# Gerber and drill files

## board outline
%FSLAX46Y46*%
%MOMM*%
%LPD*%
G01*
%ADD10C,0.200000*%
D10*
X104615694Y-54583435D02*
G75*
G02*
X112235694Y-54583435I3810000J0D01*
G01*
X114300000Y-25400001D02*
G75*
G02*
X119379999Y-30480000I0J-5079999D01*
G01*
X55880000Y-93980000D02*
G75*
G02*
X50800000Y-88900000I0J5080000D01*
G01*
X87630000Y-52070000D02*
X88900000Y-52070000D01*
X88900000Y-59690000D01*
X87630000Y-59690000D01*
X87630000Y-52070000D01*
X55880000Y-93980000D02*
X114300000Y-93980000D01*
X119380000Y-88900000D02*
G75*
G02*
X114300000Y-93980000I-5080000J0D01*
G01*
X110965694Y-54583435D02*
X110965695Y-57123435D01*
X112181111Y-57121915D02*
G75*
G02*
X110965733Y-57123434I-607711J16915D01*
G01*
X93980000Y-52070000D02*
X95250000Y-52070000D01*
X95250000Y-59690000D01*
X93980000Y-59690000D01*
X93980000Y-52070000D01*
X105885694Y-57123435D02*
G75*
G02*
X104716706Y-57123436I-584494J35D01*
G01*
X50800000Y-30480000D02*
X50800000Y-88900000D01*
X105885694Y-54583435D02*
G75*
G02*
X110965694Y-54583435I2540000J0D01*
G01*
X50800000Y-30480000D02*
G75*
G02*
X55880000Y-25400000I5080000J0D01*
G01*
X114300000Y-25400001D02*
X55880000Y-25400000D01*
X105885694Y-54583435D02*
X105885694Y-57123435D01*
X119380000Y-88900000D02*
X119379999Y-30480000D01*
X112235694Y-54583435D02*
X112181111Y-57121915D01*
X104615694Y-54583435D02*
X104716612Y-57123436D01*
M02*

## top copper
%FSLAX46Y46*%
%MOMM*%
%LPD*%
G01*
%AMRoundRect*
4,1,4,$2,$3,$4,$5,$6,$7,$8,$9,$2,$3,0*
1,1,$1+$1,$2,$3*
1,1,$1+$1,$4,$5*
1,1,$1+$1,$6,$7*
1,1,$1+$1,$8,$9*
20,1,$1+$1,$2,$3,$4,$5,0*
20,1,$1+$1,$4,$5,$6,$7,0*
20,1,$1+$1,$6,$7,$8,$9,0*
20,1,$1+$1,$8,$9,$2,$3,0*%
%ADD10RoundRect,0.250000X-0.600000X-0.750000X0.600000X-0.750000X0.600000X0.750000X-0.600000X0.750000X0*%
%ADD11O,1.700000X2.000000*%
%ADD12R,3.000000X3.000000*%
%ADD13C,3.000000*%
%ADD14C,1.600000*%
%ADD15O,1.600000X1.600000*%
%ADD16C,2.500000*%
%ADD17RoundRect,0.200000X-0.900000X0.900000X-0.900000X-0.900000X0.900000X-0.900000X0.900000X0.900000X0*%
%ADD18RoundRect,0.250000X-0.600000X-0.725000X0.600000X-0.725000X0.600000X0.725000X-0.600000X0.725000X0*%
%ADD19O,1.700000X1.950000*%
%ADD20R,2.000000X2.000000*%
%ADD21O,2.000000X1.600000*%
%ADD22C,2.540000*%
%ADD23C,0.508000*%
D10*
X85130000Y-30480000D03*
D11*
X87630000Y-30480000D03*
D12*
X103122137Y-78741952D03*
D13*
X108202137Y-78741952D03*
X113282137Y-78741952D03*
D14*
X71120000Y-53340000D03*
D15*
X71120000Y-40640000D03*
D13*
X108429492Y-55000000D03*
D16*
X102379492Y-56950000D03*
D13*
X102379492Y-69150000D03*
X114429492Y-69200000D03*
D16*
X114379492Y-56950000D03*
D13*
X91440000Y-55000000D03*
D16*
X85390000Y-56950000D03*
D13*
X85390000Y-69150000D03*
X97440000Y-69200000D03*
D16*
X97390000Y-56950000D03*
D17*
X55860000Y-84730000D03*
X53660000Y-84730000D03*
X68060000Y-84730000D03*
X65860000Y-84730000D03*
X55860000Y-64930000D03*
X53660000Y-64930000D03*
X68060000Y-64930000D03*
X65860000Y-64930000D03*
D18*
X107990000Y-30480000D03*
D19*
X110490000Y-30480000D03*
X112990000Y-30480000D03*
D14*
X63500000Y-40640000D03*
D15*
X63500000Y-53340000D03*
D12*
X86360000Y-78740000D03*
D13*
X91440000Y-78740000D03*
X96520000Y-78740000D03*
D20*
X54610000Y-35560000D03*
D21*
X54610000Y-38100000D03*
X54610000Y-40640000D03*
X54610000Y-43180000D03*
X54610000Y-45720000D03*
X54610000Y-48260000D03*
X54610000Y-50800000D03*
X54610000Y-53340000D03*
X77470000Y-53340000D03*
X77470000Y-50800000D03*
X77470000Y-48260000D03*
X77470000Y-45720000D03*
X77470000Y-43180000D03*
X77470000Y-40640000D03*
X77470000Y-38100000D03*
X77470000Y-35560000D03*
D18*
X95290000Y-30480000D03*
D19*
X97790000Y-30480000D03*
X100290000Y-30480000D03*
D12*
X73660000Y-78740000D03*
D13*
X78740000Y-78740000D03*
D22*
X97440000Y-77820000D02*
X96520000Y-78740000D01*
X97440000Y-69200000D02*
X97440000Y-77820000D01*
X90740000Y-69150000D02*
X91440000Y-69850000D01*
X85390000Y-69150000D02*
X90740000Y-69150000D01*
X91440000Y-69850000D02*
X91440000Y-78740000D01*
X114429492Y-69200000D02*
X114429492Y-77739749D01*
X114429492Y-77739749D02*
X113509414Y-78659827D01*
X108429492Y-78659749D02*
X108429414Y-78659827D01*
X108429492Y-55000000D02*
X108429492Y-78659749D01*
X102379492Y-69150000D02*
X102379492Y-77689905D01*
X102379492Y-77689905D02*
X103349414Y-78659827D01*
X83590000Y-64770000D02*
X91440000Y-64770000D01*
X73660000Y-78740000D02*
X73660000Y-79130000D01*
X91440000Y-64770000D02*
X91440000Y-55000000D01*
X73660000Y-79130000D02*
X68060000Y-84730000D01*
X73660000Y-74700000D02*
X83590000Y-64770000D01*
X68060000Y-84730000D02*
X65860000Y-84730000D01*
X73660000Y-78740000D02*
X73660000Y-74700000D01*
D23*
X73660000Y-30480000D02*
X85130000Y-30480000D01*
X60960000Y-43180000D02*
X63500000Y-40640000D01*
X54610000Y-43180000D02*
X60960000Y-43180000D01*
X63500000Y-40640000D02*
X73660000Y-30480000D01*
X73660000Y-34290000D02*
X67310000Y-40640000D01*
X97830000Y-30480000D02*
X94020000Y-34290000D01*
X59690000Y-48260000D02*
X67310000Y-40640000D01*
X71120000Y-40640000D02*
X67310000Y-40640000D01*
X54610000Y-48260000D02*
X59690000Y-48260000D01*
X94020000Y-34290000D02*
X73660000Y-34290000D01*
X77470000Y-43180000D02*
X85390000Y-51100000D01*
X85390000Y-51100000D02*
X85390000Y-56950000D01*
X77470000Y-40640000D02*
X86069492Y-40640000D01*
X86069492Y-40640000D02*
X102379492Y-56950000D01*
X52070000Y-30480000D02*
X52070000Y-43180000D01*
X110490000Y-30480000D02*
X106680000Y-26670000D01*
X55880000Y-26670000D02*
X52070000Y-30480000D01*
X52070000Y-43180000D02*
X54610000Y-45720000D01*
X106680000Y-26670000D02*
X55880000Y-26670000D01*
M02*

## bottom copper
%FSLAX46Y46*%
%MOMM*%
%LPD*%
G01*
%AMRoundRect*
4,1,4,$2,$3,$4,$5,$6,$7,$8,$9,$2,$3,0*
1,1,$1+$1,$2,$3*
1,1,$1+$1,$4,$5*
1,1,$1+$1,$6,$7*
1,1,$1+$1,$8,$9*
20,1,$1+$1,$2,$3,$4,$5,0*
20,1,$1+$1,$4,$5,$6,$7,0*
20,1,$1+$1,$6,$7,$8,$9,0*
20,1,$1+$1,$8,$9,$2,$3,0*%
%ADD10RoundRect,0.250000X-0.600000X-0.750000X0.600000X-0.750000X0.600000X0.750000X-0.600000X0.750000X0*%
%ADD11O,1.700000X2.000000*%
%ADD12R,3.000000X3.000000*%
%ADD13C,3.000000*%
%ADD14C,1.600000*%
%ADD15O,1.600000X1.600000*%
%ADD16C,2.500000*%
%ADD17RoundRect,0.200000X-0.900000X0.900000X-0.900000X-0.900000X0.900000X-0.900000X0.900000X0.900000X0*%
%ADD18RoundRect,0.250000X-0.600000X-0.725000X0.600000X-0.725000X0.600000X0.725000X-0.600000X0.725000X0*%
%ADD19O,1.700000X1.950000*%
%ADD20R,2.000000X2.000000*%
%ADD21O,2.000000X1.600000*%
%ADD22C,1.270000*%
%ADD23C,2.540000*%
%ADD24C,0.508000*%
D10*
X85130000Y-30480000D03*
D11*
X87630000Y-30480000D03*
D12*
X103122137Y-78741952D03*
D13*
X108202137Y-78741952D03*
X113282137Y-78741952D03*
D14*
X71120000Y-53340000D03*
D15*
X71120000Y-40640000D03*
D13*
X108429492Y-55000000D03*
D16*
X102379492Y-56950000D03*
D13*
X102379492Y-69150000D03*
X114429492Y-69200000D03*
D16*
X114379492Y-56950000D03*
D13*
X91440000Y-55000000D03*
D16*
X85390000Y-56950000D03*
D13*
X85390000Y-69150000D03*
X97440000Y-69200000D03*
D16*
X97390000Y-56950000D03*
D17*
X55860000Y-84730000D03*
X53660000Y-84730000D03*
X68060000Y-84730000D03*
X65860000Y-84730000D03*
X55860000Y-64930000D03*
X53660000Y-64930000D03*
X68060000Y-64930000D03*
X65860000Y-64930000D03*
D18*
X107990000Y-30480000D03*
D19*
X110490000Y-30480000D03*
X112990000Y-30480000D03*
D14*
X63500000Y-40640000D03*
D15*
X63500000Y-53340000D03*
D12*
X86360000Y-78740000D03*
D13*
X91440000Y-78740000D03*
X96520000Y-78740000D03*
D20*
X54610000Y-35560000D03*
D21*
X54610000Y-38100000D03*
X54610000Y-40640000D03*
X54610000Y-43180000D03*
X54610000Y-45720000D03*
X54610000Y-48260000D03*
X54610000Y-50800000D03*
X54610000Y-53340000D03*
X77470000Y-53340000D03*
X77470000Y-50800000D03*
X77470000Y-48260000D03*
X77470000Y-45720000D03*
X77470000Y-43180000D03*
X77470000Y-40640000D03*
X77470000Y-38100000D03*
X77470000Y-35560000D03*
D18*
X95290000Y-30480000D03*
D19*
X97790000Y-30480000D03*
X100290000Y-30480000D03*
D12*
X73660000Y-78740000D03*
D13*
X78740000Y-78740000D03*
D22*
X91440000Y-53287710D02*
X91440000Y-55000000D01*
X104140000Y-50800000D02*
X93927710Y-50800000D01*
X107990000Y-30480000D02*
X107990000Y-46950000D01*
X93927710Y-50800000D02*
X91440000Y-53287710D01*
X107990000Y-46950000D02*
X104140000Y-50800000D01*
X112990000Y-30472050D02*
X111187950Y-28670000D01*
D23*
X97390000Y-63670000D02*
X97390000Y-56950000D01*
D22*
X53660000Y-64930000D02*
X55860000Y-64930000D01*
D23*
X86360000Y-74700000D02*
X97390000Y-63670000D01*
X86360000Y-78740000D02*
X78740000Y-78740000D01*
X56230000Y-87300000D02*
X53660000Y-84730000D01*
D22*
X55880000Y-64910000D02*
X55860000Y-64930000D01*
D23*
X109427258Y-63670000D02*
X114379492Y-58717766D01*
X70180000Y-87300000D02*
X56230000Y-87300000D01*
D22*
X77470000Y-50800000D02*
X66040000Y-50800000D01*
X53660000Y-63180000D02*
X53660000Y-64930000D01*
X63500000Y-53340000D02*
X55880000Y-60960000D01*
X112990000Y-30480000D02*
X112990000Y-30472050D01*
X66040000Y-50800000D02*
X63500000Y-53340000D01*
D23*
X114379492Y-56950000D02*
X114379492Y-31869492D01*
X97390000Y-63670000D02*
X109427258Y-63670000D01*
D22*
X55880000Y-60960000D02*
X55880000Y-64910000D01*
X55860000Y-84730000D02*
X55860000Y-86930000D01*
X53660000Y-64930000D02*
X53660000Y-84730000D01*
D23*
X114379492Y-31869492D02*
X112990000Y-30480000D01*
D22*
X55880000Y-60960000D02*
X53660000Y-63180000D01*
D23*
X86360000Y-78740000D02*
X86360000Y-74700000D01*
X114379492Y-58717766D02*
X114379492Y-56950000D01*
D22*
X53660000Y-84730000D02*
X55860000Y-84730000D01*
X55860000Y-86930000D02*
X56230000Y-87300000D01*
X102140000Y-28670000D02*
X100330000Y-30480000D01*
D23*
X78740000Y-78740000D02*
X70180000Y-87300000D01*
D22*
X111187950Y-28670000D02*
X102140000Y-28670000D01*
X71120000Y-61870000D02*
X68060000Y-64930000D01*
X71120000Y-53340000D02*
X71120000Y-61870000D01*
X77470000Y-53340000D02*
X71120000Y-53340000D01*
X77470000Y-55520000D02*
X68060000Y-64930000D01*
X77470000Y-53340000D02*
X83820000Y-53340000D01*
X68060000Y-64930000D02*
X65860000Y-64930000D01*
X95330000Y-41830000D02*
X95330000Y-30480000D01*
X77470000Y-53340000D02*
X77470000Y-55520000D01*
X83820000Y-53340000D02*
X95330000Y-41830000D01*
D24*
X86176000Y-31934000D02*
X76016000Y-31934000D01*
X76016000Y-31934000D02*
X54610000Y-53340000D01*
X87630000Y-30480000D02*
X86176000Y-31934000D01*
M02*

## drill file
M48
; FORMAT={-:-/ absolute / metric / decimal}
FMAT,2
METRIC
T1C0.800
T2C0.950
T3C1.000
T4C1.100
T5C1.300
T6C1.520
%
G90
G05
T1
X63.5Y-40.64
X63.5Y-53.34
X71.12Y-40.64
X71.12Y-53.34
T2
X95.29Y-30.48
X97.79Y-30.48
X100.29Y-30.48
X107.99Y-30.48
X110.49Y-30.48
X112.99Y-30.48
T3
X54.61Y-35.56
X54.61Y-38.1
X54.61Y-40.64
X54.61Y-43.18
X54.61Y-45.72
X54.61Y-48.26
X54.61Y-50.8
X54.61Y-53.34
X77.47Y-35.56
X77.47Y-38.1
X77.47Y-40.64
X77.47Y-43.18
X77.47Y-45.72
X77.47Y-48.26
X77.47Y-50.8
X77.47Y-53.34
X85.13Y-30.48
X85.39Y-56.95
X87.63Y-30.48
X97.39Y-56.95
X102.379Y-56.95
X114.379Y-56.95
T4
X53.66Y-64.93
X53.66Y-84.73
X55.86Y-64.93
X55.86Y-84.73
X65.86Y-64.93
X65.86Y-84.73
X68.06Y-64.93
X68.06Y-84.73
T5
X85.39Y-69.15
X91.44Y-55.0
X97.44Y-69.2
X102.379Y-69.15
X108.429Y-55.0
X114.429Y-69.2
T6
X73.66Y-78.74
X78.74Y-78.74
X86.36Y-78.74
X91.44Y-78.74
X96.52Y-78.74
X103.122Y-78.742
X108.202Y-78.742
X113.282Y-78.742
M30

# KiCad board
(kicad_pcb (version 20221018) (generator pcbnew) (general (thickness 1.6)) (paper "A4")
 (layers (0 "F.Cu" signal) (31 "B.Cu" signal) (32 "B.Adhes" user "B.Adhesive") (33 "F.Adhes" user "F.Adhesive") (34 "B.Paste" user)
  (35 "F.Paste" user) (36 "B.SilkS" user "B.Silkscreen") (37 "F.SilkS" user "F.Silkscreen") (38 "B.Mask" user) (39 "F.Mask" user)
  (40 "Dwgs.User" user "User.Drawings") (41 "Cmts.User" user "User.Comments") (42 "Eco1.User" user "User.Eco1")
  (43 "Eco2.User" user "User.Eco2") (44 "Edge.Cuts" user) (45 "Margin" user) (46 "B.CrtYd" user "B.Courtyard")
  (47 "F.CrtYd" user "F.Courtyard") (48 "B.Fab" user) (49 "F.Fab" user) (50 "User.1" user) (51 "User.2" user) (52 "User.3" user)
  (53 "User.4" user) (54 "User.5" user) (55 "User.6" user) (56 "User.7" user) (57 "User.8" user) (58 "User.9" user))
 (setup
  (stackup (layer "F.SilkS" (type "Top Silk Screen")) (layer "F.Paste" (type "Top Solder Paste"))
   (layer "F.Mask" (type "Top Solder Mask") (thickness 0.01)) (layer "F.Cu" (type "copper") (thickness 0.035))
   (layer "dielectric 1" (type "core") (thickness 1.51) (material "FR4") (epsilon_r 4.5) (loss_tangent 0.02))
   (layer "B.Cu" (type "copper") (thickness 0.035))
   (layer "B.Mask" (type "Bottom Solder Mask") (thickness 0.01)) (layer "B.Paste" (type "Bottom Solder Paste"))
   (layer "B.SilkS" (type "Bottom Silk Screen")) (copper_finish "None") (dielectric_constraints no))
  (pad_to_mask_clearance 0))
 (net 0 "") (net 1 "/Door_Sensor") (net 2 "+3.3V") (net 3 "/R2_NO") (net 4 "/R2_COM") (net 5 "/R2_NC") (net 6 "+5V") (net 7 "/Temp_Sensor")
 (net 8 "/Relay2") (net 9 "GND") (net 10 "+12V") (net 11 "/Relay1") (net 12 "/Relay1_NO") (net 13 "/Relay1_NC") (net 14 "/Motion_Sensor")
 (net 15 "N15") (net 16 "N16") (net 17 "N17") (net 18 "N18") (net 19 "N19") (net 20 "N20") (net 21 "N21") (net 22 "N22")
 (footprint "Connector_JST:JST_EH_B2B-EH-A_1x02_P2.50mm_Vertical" (layer "F.Cu") (at 85.13 30.48)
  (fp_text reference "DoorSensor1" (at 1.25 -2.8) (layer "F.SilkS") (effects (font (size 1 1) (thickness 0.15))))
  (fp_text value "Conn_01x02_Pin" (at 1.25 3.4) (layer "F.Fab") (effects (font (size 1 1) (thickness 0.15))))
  (pad "1" thru_hole roundrect (at 0 0) (size 1.7 2) (drill 1) (layers "*.Cu" "*.Mask") (roundrect_rratio 0.1470588235)
   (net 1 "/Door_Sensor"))
  (pad "2" thru_hole oval (at 2.5 0) (size 1.7 2) (drill 1) (layers "*.Cu" "*.Mask") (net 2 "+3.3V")))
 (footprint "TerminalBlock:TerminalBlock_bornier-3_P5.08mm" (layer "F.Cu") (at 103.122137 78.741952)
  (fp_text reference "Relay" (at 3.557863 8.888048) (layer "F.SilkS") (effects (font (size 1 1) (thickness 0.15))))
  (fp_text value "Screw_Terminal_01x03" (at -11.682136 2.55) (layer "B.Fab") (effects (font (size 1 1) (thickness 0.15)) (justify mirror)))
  (pad "1" thru_hole rect (at 0 0) (size 3 3) (drill 1.52) (layers "*.Cu" "*.Mask") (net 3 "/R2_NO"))
  (pad "2" thru_hole circle (at 5.08 0) (size 3 3) (drill 1.52) (layers "*.Cu" "*.Mask") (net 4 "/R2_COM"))
  (pad "3" thru_hole circle (at 10.16 0) (size 3 3) (drill 1.52) (layers "*.Cu" "*.Mask") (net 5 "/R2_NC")))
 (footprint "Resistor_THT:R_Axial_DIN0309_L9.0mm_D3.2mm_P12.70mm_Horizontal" (layer "F.Cu") (at 71.12 53.34 90)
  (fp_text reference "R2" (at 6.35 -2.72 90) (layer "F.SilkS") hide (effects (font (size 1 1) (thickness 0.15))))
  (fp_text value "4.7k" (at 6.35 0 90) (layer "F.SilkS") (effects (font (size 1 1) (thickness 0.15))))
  (pad "1" thru_hole circle (at 0 0 90) (size 1.6 1.6) (drill 0.8) (layers "*.Cu" "*.Mask") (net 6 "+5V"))
  (pad "2" thru_hole oval (at 12.7 0 90) (size 1.6 1.6) (drill 0.8) (layers "*.Cu" "*.Mask") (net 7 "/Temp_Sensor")))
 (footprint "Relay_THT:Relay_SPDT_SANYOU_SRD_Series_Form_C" (layer "F.Cu") (at 108.429492 55 -90)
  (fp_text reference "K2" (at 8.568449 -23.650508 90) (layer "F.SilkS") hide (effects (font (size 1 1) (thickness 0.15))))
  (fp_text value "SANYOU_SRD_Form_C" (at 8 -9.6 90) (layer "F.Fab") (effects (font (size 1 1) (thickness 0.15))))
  (pad "1" thru_hole circle (at 0 0) (size 3 3) (drill 1.3) (layers "*.Cu" "*.Mask") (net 4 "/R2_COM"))
  (pad "2" thru_hole circle (at 1.95 6.05) (size 2.5 2.5) (drill 1) (layers "*.Cu" "*.Mask") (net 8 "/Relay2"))
  (pad "3" thru_hole circle (at 14.15 6.05) (size 3 3) (drill 1.3) (layers "*.Cu" "*.Mask") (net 3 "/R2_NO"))
  (pad "4" thru_hole circle (at 14.2 -6) (size 3 3) (drill 1.3) (layers "*.Cu" "*.Mask") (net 5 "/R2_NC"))
  (pad "5" thru_hole circle (at 1.95 -5.95) (size 2.5 2.5) (drill 1) (layers "*.Cu" "*.Mask") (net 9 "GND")))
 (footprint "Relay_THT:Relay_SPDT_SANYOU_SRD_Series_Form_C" (layer "F.Cu") (at 91.44 55 -90)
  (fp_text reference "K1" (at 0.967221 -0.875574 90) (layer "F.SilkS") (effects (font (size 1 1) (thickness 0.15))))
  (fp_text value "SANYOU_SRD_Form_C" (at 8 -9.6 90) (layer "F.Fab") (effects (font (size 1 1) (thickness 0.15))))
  (pad "1" thru_hole circle (at 0 0) (size 3 3) (drill 1.3) (layers "*.Cu" "*.Mask") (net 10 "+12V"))
  (pad "2" thru_hole circle (at 1.95 6.05) (size 2.5 2.5) (drill 1) (layers "*.Cu" "*.Mask") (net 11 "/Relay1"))
  (pad "3" thru_hole circle (at 14.15 6.05) (size 3 3) (drill 1.3) (layers "*.Cu" "*.Mask") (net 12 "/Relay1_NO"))
  (pad "4" thru_hole circle (at 14.2 -6) (size 3 3) (drill 1.3) (layers "*.Cu" "*.Mask") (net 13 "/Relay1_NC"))
  (pad "5" thru_hole circle (at 1.95 -5.95) (size 2.5 2.5) (drill 1) (layers "*.Cu" "*.Mask") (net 9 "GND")))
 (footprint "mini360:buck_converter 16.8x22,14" (layer "F.Cu") (at 60.96 74.93 -90)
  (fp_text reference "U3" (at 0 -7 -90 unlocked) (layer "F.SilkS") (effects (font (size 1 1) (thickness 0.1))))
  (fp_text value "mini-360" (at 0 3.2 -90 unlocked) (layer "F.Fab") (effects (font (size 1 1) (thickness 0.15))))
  (pad "1" thru_hole roundrect (at 9.8 5.1 270) (size 2.2 2.2) (drill 1.1) (layers "*.Cu" "*.Mask") (roundrect_rratio 0.09090909091)
   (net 9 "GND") (thermal_bridge_angle 45))
  (pad "1" thru_hole roundrect (at 9.8 7.3 270) (size 2.2 2.2) (drill 1.1) (layers "*.Cu" "*.Mask") (roundrect_rratio 0.09090909091)
   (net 9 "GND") (thermal_bridge_angle 45))
  (pad "2" thru_hole roundrect (at 9.8 -7.1 270) (size 2.2 2.2) (drill 1.1) (layers "*.Cu" "*.Mask") (roundrect_rratio 0.09090909091)
   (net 10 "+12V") (thermal_bridge_angle 45))
  (pad "2" thru_hole roundrect (at 9.8 -4.9 270) (size 2.2 2.2) (drill 1.1) (layers "*.Cu" "*.Mask") (roundrect_rratio 0.09090909091)
   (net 10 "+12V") (thermal_bridge_angle 45))
  (pad "3" thru_hole roundrect (at -10 5.1 270) (size 2.2 2.2) (drill 1.1) (layers "*.Cu" "*.Mask") (roundrect_rratio 0.09090909091)
   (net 9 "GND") (thermal_bridge_angle 45))
  (pad "3" thru_hole roundrect (at -10 7.3 270) (size 2.2 2.2) (drill 1.1) (layers "*.Cu" "*.Mask") (roundrect_rratio 0.09090909091)
   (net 9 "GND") (thermal_bridge_angle 45))
  (pad "4" thru_hole roundrect (at -10 -7.1 270) (size 2.2 2.2) (drill 1.1) (layers "*.Cu" "*.Mask") (roundrect_rratio 0.09090909091)
   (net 6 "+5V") (thermal_bridge_angle 45))
  (pad "4" thru_hole roundrect (at -10 -4.9 270) (size 2.2 2.2) (drill 1.1) (layers "*.Cu" "*.Mask") (roundrect_rratio 0.09090909091)
   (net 6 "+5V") (thermal_bridge_angle 45)))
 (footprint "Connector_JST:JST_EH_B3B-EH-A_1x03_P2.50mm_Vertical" (layer "F.Cu") (at 107.99 30.48)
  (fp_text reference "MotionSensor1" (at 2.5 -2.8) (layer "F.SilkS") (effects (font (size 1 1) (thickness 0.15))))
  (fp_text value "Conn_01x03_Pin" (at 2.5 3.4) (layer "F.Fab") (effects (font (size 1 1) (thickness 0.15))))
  (pad "1" thru_hole roundrect (at 0 0) (size 1.7 1.95) (drill 0.95) (layers "*.Cu" "*.Mask") (roundrect_rratio 0.1470588235)
   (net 10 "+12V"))
  (pad "2" thru_hole oval (at 2.5 0) (size 1.7 1.95) (drill 0.95) (layers "*.Cu" "*.Mask") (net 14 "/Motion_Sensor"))
  (pad "3" thru_hole oval (at 5 0) (size 1.7 1.95) (drill 0.95) (layers "*.Cu" "*.Mask") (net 9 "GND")))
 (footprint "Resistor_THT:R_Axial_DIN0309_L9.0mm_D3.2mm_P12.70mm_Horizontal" (layer "F.Cu") (at 63.5 40.64 -90)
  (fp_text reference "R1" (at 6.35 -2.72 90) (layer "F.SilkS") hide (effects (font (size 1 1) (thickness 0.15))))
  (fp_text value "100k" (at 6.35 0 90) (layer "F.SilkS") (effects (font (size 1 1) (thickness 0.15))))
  (pad "1" thru_hole circle (at 0 0 270) (size 1.6 1.6) (drill 0.8) (layers "*.Cu" "*.Mask") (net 1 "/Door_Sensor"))
  (pad "2" thru_hole oval (at 12.7 0 270) (size 1.6 1.6) (drill 0.8) (layers "*.Cu" "*.Mask") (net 9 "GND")))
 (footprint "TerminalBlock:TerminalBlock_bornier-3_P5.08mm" (layer "F.Cu") (at 86.36 78.74)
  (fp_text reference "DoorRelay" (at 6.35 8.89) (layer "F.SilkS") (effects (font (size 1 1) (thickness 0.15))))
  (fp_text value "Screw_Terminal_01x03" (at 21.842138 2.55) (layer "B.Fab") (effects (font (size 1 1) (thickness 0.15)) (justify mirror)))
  (pad "1" thru_hole rect (at 0 0) (size 3 3) (drill 1.52) (layers "*.Cu" "*.Mask") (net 9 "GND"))
  (pad "2" thru_hole circle (at 5.08 0) (size 3 3) (drill 1.52) (layers "*.Cu" "*.Mask") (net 12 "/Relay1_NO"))
  (pad "3" thru_hole circle (at 10.16 0) (size 3 3) (drill 1.52) (layers "*.Cu" "*.Mask") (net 13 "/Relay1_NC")))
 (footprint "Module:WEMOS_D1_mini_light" (layer "F.Cu") (at 54.61 35.56)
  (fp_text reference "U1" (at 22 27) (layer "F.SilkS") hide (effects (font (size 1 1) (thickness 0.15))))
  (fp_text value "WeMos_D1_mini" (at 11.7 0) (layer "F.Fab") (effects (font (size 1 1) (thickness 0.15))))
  (pad "1" thru_hole rect (at 0 0) (size 2 2) (drill 1) (layers "*.Cu" "*.Mask") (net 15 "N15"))
  (pad "2" thru_hole oval (at 0 2.54) (size 2 1.6) (drill 1) (layers "*.Cu" "*.Mask") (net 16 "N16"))
  (pad "3" thru_hole oval (at 0 5.08) (size 2 1.6) (drill 1) (layers "*.Cu" "*.Mask") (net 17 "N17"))
  (pad "4" thru_hole oval (at 0 7.62) (size 2 1.6) (drill 1) (layers "*.Cu" "*.Mask") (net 1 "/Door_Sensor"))
  (pad "5" thru_hole oval (at 0 10.16) (size 2 1.6) (drill 1) (layers "*.Cu" "*.Mask") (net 14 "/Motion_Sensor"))
  (pad "6" thru_hole oval (at 0 12.7) (size 2 1.6) (drill 1) (layers "*.Cu" "*.Mask") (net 7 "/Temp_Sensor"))
  (pad "7" thru_hole oval (at 0 15.24) (size 2 1.6) (drill 1) (layers "*.Cu" "*.Mask") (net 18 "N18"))
  (pad "8" thru_hole oval (at 0 17.78) (size 2 1.6) (drill 1) (layers "*.Cu" "*.Mask") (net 2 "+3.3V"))
  (pad "9" thru_hole oval (at 22.86 17.78) (size 2 1.6) (drill 1) (layers "*.Cu" "*.Mask") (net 6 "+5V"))
  (pad "10" thru_hole oval (at 22.86 15.24) (size 2 1.6) (drill 1) (layers "*.Cu" "*.Mask") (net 9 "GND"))
  (pad "11" thru_hole oval (at 22.86 12.7) (size 2 1.6) (drill 1) (layers "*.Cu" "*.Mask") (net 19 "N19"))
  (pad "12" thru_hole oval (at 22.86 10.16) (size 2 1.6) (drill 1) (layers "*.Cu" "*.Mask") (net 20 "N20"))
  (pad "13" thru_hole oval (at 22.86 7.62) (size 2 1.6) (drill 1) (layers "*.Cu" "*.Mask") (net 11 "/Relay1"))
  (pad "14" thru_hole oval (at 22.86 5.08) (size 2 1.6) (drill 1) (layers "*.Cu" "*.Mask") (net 8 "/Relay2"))
  (pad "15" thru_hole oval (at 22.86 2.54) (size 2 1.6) (drill 1) (layers "*.Cu" "*.Mask") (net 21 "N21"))
  (pad "16" thru_hole oval (at 22.86 0) (size 2 1.6) (drill 1) (layers "*.Cu" "*.Mask") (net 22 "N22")))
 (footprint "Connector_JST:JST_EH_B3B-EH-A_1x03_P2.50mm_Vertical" (layer "F.Cu") (at 95.29 30.48)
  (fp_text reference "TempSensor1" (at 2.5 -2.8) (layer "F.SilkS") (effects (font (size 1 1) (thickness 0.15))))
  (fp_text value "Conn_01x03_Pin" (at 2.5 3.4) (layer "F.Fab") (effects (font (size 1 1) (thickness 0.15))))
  (pad "1" thru_hole roundrect (at 0 0) (size 1.7 1.95) (drill 0.95) (layers "*.Cu" "*.Mask") (roundrect_rratio 0.1470588235) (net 6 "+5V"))
  (pad "2" thru_hole oval (at 2.5 0) (size 1.7 1.95) (drill 0.95) (layers "*.Cu" "*.Mask") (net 7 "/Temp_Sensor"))
  (pad "3" thru_hole oval (at 5 0) (size 1.7 1.95) (drill 0.95) (layers "*.Cu" "*.Mask") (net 9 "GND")))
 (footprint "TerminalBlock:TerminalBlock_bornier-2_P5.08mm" (layer "F.Cu") (at 73.66 78.74)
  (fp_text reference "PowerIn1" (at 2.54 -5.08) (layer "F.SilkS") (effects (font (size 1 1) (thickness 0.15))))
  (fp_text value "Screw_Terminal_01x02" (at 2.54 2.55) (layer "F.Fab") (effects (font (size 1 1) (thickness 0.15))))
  (pad "1" thru_hole rect (at 0 0) (size 3 3) (drill 1.52) (layers "*.Cu" "*.Mask") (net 10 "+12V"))
  (pad "2" thru_hole circle (at 5.08 0) (size 3 3) (drill 1.52) (layers "*.Cu" "*.Mask") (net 9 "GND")))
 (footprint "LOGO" (layer "B.Cu") (at 67.31 59.69 180)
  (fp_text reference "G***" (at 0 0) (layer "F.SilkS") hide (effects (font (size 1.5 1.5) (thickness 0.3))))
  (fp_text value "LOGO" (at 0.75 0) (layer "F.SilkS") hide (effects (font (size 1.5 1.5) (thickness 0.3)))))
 (gr_arc (start 104.615694 54.583435) (mid 108.425694 50.773435) (end 112.235694 54.583435) (stroke (width 0.2) (type default))
  (layer "Edge.Cuts"))
 (gr_arc (start 114.3 25.400001) (mid 117.892102 26.887898) (end 119.379999 30.48) (stroke (width 0.2) (type default)) (layer "Edge.Cuts"))
 (gr_arc (start 55.88 93.98) (mid 52.287898 92.492102) (end 50.8 88.9) (stroke (width 0.2) (type default)) (layer "Edge.Cuts"))
 (gr_rect (start 87.63 52.07) (end 88.9 59.69) (stroke (width 0.2) (type default)) (fill none) (layer "Edge.Cuts"))
 (gr_line (start 55.88 93.98) (end 114.3 93.98) (stroke (width 0.2) (type default)) (layer "Edge.Cuts"))
 (gr_arc (start 119.38 88.9) (mid 117.892102 92.492102) (end 114.3 93.98) (stroke (width 0.2) (type default)) (layer "Edge.Cuts"))
 (gr_line (start 110.965694 54.583435) (end 110.965695 57.123435) (stroke (width 0.2) (type default)) (layer "Edge.Cuts"))
 (gr_arc (start 112.181111 57.121915) (mid 111.574141 57.712966) (end 110.965695 57.123435) (stroke (width 0.2) (type default))
  (layer "Edge.Cuts"))
 (gr_rect (start 93.98 52.07) (end 95.25 59.69) (stroke (width 0.2) (type default)) (fill none) (layer "Edge.Cuts"))
 (gr_arc (start 105.885694 57.123435) (mid 105.301153 57.707941) (end 104.716612 57.123436) (stroke (width 0.2) (type default))
  (layer "Edge.Cuts"))
 (gr_line (start 50.8 30.48) (end 50.8 88.9) (stroke (width 0.2) (type default)) (layer "Edge.Cuts"))
 (gr_arc (start 105.885694 54.583435) (mid 108.425694 52.043435) (end 110.965694 54.583435) (stroke (width 0.2) (type default))
  (layer "Edge.Cuts"))
 (gr_arc (start 50.8 30.48) (mid 52.287898 26.887898) (end 55.88 25.4) (stroke (width 0.2) (type default)) (layer "Edge.Cuts"))
 (gr_line (start 114.3 25.400001) (end 55.88 25.4) (stroke (width 0.2) (type default)) (layer "Edge.Cuts"))
 (gr_line (start 105.885694 54.583435) (end 105.885694 57.123435) (stroke (width 0.2) (type default)) (layer "Edge.Cuts"))
 (gr_line (start 119.38 88.9) (end 119.379999 30.48) (stroke (width 0.2) (type default)) (layer "Edge.Cuts"))
 (gr_line (start 112.235694 54.583435) (end 112.181111 57.121915) (stroke (width 0.2) (type default)) (layer "Edge.Cuts"))
 (gr_line (start 104.615694 54.583435) (end 104.716612 57.123436) (stroke (width 0.2) (type default)) (layer "Edge.Cuts"))
 (segment (start 97.44 77.82) (end 96.52 78.74) (width 2.54) (layer "F.Cu") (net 13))
 (segment (start 97.44 69.2) (end 97.44 77.82) (width 2.54) (layer "F.Cu") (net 13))
 (segment (start 90.74 69.15) (end 91.44 69.85) (width 2.54) (layer "F.Cu") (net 12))
 (segment (start 85.39 69.15) (end 90.74 69.15) (width 2.54) (layer "F.Cu") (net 12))
 (segment (start 91.44 69.85) (end 91.44 78.74) (width 2.54) (layer "F.Cu") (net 12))
 (segment (start 114.429492 69.2) (end 114.429492 77.739749) (width 2.54) (layer "F.Cu") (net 5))
 (segment (start 114.429492 77.739749) (end 113.509414 78.659827) (width 2.54) (layer "F.Cu") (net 5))
 (segment (start 108.429492 78.659749) (end 108.429414 78.659827) (width 2.54) (layer "F.Cu") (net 4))
 (segment (start 108.429492 55) (end 108.429492 78.659749) (width 2.54) (layer "F.Cu") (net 4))
 (segment (start 102.379492 69.15) (end 102.379492 77.689905) (width 2.54) (layer "F.Cu") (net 3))
 (segment (start 102.379492 77.689905) (end 103.349414 78.659827) (width 2.54) (layer "F.Cu") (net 3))
 (segment (start 83.59 64.77) (end 91.44 64.77) (width 2.54) (layer "F.Cu") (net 10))
 (segment (start 73.66 78.74) (end 73.66 79.13) (width 2.54) (layer "F.Cu") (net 10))
 (segment (start 91.44 64.77) (end 91.44 55) (width 2.54) (layer "F.Cu") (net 10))
 (segment (start 73.66 79.13) (end 68.06 84.73) (width 2.54) (layer "F.Cu") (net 10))
 (segment (start 73.66 74.7) (end 83.59 64.77) (width 2.54) (layer "F.Cu") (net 10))
 (segment (start 68.06 84.73) (end 65.86 84.73) (width 2.54) (layer "F.Cu") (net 10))
 (segment (start 73.66 78.74) (end 73.66 74.7) (width 2.54) (layer "F.Cu") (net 10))
 (segment (start 91.44 53.28771) (end 91.44 55) (width 1.27) (layer "B.Cu") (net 10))
 (segment (start 104.14 50.8) (end 93.92771 50.8) (width 1.27) (layer "B.Cu") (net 10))
 (segment (start 107.99 30.48) (end 107.99 46.95) (width 1.27) (layer "B.Cu") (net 10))
 (segment (start 93.92771 50.8) (end 91.44 53.28771) (width 1.27) (layer "B.Cu") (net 10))
 (segment (start 107.99 46.95) (end 104.14 50.8) (width 1.27) (layer "B.Cu") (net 10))
 (segment (start 112.99 30.47205) (end 111.18795 28.67) (width 1.27) (layer "B.Cu") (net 9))
 (segment (start 97.39 63.67) (end 97.39 56.95) (width 2.54) (layer "B.Cu") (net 9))
 (segment (start 53.66 64.93) (end 55.86 64.93) (width 1.27) (layer "B.Cu") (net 9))
 (segment (start 86.36 74.7) (end 97.39 63.67) (width 2.54) (layer "B.Cu") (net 9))
 (segment (start 86.36 78.74) (end 78.74 78.74) (width 2.54) (layer "B.Cu") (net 9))
 (segment (start 56.23 87.3) (end 53.66 84.73) (width 2.54) (layer "B.Cu") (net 9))
 (segment (start 55.88 64.91) (end 55.86 64.93) (width 1.27) (layer "B.Cu") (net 9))
 (segment (start 109.427258 63.67) (end 114.379492 58.717766) (width 2.54) (layer "B.Cu") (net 9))
 (segment (start 70.18 87.3) (end 56.23 87.3) (width 2.54) (layer "B.Cu") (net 9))
 (segment (start 77.47 50.8) (end 66.04 50.8) (width 1.27) (layer "B.Cu") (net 9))
 (segment (start 53.66 63.18) (end 53.66 64.93) (width 1.27) (layer "B.Cu") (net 9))
 (segment (start 63.5 53.34) (end 55.88 60.96) (width 1.27) (layer "B.Cu") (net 9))
 (segment (start 112.99 30.48) (end 112.99 30.47205) (width 1.27) (layer "B.Cu") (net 9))
 (segment (start 66.04 50.8) (end 63.5 53.34) (width 1.27) (layer "B.Cu") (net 9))
 (segment (start 114.379492 56.95) (end 114.379492 31.869492) (width 2.54) (layer "B.Cu") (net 9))
 (segment (start 97.39 63.67) (end 109.427258 63.67) (width 2.54) (layer "B.Cu") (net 9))
 (segment (start 55.88 60.96) (end 55.88 64.91) (width 1.27) (layer "B.Cu") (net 9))
 (segment (start 55.86 84.73) (end 55.86 86.93) (width 1.27) (layer "B.Cu") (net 9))
 (segment (start 53.66 64.93) (end 53.66 84.73) (width 1.27) (layer "B.Cu") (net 9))
 (segment (start 114.379492 31.869492) (end 112.99 30.48) (width 2.54) (layer "B.Cu") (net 9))
 (segment (start 55.88 60.96) (end 53.66 63.18) (width 1.27) (layer "B.Cu") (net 9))
 (segment (start 86.36 78.74) (end 86.36 74.7) (width 2.54) (layer "B.Cu") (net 9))
 (segment (start 114.379492 58.717766) (end 114.379492 56.95) (width 2.54) (layer "B.Cu") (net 9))
 (segment (start 53.66 84.73) (end 55.86 84.73) (width 1.27) (layer "B.Cu") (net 9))
 (segment (start 55.86 86.93) (end 56.23 87.3) (width 1.27) (layer "B.Cu") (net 9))
 (segment (start 102.14 28.67) (end 100.33 30.48) (width 1.27) (layer "B.Cu") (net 9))
 (segment (start 78.74 78.74) (end 70.18 87.3) (width 2.54) (layer "B.Cu") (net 9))
 (segment (start 111.18795 28.67) (end 102.14 28.67) (width 1.27) (layer "B.Cu") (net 9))
 (segment (start 73.66 30.48) (end 85.13 30.48) (width 0.508) (layer "F.Cu") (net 1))
 (segment (start 60.96 43.18) (end 63.5 40.64) (width 0.508) (layer "F.Cu") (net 1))
 (segment (start 54.61 43.18) (end 60.96 43.18) (width 0.508) (layer "F.Cu") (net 1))
 (segment (start 63.5 40.64) (end 73.66 30.48) (width 0.508) (layer "F.Cu") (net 1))
 (segment (start 71.12 61.87) (end 68.06 64.93) (width 1.27) (layer "B.Cu") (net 6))
 (segment (start 71.12 53.34) (end 71.12 61.87) (width 1.27) (layer "B.Cu") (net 6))
 (segment (start 77.47 53.34) (end 71.12 53.34) (width 1.27) (layer "B.Cu") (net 6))
 (segment (start 77.47 55.52) (end 68.06 64.93) (width 1.27) (layer "B.Cu") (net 6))
 (segment (start 77.47 53.34) (end 83.82 53.34) (width 1.27) (layer "B.Cu") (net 6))
 (segment (start 68.06 64.93) (end 65.86 64.93) (width 1.27) (layer "B.Cu") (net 6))
 (segment (start 95.33 41.83) (end 95.33 30.48) (width 1.27) (layer "B.Cu") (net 6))
 (segment (start 77.47 53.34) (end 77.47 55.52) (width 1.27) (layer "B.Cu") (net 6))
 (segment (start 83.82 53.34) (end 95.33 41.83) (width 1.27) (layer "B.Cu") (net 6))
 (segment (start 73.66 34.29) (end 67.31 40.64) (width 0.508) (layer "F.Cu") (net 7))
 (segment (start 97.83 30.48) (end 94.02 34.29) (width 0.508) (layer "F.Cu") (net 7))
 (segment (start 59.69 48.26) (end 67.31 40.64) (width 0.508) (layer "F.Cu") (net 7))
 (segment (start 71.12 40.64) (end 67.31 40.64) (width 0.508) (layer "F.Cu") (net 7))
 (segment (start 54.61 48.26) (end 59.69 48.26) (width 0.508) (layer "F.Cu") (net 7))
 (segment (start 94.02 34.29) (end 73.66 34.29) (width 0.508) (layer "F.Cu") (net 7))
 (segment (start 77.47 43.18) (end 85.39 51.1) (width 0.508) (layer "F.Cu") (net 11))
 (segment (start 85.39 51.1) (end 85.39 56.95) (width 0.508) (layer "F.Cu") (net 11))
 (segment (start 77.47 40.64) (end 86.069492 40.64) (width 0.508) (layer "F.Cu") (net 8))
 (segment (start 86.069492 40.64) (end 102.379492 56.95) (width 0.508) (layer "F.Cu") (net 8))
 (segment (start 86.176 31.934) (end 76.016 31.934) (width 0.508) (layer "B.Cu") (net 2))
 (segment (start 76.016 31.934) (end 54.61 53.34) (width 0.508) (layer "B.Cu") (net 2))
 (segment (start 87.63 30.48) (end 86.176 31.934) (width 0.508) (layer "B.Cu") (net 2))
 (segment (start 52.07 30.48) (end 52.07 43.18) (width 0.508) (layer "F.Cu") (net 14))
 (segment (start 110.49 30.48) (end 106.68 26.67) (width 0.508) (layer "F.Cu") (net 14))
 (segment (start 55.88 26.67) (end 52.07 30.48) (width 0.508) (layer "F.Cu") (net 14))
 (segment (start 52.07 43.18) (end 54.61 45.72) (width 0.508) (layer "F.Cu") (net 14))
 (segment (start 106.68 26.67) (end 55.88 26.67) (width 0.508) (layer "F.Cu") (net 14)))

